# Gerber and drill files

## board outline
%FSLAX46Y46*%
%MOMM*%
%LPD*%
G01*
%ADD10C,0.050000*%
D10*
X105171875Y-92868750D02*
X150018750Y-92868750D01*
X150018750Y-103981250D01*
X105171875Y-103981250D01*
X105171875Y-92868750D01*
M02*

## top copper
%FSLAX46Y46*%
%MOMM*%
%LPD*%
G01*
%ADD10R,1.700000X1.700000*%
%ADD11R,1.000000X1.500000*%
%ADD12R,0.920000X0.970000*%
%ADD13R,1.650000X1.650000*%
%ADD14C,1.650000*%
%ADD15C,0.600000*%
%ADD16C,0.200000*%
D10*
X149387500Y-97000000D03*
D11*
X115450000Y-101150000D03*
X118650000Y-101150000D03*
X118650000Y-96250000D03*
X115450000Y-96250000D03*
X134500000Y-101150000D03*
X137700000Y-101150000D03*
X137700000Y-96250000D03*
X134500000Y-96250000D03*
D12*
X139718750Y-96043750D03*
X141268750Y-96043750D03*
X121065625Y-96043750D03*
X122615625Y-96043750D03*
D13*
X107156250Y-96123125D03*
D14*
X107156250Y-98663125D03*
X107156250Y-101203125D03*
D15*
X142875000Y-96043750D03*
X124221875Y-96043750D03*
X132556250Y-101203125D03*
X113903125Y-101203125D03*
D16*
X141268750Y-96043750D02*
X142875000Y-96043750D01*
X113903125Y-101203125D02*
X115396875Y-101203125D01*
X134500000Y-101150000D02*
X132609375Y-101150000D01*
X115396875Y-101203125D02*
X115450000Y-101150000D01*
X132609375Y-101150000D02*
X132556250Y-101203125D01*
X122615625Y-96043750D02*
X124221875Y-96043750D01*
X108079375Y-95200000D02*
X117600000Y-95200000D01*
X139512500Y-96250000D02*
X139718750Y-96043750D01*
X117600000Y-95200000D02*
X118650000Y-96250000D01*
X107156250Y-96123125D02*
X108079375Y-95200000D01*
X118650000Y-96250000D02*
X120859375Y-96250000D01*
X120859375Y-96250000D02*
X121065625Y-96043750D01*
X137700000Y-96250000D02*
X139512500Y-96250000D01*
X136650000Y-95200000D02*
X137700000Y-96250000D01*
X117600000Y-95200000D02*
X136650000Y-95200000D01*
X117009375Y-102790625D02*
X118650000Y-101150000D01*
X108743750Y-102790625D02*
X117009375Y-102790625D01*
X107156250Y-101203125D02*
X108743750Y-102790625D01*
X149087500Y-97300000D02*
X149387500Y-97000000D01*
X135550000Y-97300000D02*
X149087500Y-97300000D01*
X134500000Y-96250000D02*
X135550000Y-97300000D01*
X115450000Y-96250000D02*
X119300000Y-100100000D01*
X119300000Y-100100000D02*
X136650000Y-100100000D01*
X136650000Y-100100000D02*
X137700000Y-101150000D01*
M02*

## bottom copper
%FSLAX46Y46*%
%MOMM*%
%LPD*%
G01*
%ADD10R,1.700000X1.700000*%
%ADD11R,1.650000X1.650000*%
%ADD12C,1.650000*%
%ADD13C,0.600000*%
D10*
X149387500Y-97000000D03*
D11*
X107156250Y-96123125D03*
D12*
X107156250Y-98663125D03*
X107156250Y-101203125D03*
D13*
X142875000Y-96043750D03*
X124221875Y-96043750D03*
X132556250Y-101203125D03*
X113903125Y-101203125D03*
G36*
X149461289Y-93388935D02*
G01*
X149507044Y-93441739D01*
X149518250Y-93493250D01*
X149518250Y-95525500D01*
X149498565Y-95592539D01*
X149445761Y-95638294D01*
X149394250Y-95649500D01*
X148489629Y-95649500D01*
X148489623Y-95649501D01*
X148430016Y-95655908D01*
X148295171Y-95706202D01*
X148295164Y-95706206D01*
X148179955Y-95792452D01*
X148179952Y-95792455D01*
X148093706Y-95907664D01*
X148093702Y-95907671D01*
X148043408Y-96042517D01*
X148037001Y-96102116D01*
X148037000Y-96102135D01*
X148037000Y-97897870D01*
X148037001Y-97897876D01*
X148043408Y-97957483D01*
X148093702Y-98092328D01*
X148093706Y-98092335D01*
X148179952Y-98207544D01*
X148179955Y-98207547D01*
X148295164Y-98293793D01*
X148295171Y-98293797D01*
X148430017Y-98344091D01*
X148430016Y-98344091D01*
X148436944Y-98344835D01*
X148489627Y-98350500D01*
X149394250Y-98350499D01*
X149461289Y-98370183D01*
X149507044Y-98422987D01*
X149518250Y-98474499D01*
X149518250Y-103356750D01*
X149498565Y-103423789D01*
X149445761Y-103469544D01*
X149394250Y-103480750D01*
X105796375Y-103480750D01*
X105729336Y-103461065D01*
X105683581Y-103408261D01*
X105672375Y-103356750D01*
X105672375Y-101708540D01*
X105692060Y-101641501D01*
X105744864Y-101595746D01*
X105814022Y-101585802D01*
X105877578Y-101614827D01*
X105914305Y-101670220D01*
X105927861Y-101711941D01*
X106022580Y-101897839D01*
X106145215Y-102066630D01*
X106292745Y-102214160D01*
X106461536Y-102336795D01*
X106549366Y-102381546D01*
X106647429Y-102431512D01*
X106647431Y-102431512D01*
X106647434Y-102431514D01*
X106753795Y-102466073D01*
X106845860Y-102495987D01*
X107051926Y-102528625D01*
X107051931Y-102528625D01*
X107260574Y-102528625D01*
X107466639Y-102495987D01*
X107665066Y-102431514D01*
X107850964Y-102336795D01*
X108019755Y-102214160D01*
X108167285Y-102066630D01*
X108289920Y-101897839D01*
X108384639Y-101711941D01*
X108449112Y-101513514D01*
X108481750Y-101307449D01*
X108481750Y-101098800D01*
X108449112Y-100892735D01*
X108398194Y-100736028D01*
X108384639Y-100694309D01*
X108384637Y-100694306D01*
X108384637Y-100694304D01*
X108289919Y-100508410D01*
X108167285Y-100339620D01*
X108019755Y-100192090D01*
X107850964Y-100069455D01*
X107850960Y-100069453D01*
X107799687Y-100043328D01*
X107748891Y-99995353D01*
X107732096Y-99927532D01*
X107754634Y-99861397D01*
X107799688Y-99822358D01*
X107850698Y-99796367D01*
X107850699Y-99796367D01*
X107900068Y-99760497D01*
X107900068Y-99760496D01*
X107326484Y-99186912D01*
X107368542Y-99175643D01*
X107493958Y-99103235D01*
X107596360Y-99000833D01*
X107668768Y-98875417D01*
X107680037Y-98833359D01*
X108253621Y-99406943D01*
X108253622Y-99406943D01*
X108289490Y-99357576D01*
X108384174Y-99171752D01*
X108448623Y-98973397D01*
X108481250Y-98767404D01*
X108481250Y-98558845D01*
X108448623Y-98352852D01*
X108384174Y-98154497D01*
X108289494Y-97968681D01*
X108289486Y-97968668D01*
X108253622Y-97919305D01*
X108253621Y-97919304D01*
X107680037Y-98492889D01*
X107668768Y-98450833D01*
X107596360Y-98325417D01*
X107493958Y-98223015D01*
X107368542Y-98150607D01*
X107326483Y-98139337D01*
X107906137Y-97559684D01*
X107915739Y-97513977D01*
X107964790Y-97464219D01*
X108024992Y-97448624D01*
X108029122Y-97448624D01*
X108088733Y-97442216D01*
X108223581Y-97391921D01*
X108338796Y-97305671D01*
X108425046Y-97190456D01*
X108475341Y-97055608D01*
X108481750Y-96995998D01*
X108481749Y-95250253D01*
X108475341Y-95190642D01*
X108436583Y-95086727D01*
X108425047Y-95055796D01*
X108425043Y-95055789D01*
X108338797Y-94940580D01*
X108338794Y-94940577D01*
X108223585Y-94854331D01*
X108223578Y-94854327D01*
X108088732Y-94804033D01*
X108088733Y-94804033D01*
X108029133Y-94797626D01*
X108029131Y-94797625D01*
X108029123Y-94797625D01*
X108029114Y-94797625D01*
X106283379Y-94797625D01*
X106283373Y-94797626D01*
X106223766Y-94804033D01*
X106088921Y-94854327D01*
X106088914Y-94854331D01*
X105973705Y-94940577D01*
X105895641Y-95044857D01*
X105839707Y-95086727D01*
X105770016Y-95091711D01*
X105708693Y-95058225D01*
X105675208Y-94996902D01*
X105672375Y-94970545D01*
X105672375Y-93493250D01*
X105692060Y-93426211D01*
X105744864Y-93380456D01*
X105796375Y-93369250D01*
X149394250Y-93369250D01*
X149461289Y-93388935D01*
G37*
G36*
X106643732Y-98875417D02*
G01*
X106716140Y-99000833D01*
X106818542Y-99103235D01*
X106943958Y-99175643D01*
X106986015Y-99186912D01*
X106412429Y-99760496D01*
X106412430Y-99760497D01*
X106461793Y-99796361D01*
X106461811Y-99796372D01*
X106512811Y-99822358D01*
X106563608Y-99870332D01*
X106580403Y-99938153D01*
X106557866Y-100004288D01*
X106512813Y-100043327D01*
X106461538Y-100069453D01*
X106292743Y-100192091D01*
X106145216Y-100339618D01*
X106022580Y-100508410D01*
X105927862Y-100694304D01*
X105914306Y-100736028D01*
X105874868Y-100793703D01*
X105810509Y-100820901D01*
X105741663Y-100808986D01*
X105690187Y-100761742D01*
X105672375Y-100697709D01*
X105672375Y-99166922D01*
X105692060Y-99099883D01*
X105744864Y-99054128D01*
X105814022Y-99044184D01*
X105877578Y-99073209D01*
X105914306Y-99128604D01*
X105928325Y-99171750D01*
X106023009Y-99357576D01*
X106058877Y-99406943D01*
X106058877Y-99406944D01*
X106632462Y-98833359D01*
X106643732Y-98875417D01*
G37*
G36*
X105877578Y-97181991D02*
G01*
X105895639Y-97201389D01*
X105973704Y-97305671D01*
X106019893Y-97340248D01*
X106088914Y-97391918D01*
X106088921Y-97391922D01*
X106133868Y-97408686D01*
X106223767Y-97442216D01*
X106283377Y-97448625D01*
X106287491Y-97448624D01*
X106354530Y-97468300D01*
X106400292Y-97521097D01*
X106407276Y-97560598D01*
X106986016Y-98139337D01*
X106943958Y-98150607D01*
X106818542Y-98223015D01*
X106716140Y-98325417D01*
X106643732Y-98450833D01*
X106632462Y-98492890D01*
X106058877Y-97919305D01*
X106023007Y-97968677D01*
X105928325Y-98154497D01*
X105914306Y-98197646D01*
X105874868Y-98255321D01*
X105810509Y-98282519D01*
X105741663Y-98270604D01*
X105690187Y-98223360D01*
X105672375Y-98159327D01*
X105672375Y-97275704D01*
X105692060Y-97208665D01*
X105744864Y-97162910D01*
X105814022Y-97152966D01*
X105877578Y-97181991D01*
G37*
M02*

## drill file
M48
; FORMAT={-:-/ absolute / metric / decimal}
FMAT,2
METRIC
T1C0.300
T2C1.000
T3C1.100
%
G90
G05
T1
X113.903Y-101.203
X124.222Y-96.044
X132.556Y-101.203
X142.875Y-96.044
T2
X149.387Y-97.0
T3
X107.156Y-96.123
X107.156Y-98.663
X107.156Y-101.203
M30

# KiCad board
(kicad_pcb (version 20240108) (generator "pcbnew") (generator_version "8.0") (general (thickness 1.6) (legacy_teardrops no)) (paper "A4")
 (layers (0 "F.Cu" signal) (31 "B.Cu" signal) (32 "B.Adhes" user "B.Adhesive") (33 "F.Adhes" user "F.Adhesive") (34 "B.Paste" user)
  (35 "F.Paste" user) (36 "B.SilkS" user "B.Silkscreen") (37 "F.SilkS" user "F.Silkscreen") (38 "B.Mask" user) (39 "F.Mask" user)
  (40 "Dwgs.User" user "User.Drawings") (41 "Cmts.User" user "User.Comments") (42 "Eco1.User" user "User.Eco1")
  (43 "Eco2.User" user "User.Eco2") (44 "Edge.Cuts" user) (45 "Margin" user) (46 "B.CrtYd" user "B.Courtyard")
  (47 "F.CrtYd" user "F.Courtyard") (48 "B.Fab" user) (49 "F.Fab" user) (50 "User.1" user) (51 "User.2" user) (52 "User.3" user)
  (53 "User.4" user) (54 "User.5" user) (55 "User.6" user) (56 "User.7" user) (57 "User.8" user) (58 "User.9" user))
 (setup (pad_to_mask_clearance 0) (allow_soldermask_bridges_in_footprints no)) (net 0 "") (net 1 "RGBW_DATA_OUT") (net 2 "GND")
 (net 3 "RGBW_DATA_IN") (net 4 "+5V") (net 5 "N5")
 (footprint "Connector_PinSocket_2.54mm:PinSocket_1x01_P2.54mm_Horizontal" (layer "F.Cu") (at 149.3875 97 180)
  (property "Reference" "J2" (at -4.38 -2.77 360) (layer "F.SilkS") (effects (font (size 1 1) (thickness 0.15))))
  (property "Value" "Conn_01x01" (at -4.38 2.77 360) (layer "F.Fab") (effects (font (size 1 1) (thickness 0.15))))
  (pad "1" thru_hole rect (at 0 0 180) (size 1.7 1.7) (drill 1) (layers "*.Cu" "*.Mask") (remove_unused_layers no) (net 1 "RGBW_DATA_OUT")))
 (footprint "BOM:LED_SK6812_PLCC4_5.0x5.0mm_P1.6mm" (layer "F.Cu") (at 117.05 98.7 -90)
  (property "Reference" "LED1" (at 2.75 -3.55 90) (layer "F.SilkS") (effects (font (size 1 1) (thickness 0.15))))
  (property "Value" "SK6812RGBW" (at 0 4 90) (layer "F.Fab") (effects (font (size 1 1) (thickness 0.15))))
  (pad "1" smd rect (at 2.45 1.6 270) (size 1.5 1) (layers "F.Cu" "F.Paste" "F.Mask") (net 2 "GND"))
  (pad "2" smd rect (at 2.45 -1.6 270) (size 1.5 1) (layers "F.Cu" "F.Paste" "F.Mask") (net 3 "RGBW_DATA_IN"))
  (pad "3" smd rect (at -2.45 -1.6 270) (size 1.5 1) (layers "F.Cu" "F.Paste" "F.Mask") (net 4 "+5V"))
  (pad "4" smd rect (at -2.45 1.6 270) (size 1.5 1) (layers "F.Cu" "F.Paste" "F.Mask") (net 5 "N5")))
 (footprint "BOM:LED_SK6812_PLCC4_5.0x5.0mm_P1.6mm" (layer "F.Cu") (at 136.1 98.7 -90)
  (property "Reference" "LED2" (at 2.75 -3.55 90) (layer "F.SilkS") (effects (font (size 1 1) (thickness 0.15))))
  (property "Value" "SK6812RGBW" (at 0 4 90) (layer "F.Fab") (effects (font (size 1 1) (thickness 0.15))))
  (pad "1" smd rect (at 2.45 1.6 270) (size 1.5 1) (layers "F.Cu" "F.Paste" "F.Mask") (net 2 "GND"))
  (pad "2" smd rect (at 2.45 -1.6 270) (size 1.5 1) (layers "F.Cu" "F.Paste" "F.Mask") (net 5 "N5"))
  (pad "3" smd rect (at -2.45 -1.6 270) (size 1.5 1) (layers "F.Cu" "F.Paste" "F.Mask") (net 4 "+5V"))
  (pad "4" smd rect (at -2.45 1.6 270) (size 1.5 1) (layers "F.Cu" "F.Paste" "F.Mask") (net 1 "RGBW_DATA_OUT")))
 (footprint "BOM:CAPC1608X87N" (layer "F.Cu") (at 140.49375 96.04375)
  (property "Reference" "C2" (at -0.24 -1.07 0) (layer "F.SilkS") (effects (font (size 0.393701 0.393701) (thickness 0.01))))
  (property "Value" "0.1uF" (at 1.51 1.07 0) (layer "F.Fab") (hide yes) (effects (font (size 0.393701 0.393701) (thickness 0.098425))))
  (pad "1" smd rect (at -0.775 0) (size 0.92 0.97) (layers "F.Cu" "F.Paste" "F.Mask") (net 4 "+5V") (solder_mask_margin 0.102))
  (pad "2" smd rect (at 0.775 0) (size 0.92 0.97) (layers "F.Cu" "F.Paste" "F.Mask") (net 2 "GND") (solder_mask_margin 0.102)))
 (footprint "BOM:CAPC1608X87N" (layer "F.Cu") (at 121.840625 96.04375)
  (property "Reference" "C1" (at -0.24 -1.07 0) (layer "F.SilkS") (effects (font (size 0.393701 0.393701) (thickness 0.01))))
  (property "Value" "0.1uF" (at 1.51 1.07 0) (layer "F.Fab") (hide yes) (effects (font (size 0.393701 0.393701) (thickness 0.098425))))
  (pad "1" smd rect (at -0.775 0) (size 0.92 0.97) (layers "F.Cu" "F.Paste" "F.Mask") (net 4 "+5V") (solder_mask_margin 0.102))
  (pad "2" smd rect (at 0.775 0) (size 0.92 0.97) (layers "F.Cu" "F.Paste" "F.Mask") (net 2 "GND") (solder_mask_margin 0.102)))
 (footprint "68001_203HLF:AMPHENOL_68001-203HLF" (layer "F.Cu") (at 107.15625 98.663125 -90)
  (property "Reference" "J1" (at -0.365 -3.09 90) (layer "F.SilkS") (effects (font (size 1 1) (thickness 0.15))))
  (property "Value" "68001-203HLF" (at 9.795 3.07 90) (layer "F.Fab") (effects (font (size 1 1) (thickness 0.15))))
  (pad "01" thru_hole rect (at -2.54 0 270) (size 1.65 1.65) (drill 1.1) (layers "*.Cu" "*.Mask") (remove_unused_layers no) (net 4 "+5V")
   (solder_mask_margin 0.102))
  (pad "02" thru_hole circle (at 0 0 270) (size 1.65 1.65) (drill 1.1) (layers "*.Cu" "*.Mask") (remove_unused_layers no) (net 2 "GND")
   (solder_mask_margin 0.102))
  (pad "03" thru_hole circle (at 2.54 0 270) (size 1.65 1.65) (drill 1.1) (layers "*.Cu" "*.Mask") (remove_unused_layers no)
   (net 3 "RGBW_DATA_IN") (solder_mask_margin 0.102)))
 (gr_rect (start 105.171875 92.86875) (end 150.01875 103.98125) (stroke (width 0.05) (type default)) (fill none) (layer "Edge.Cuts"))
 (segment (start 141.26875 96.04375) (end 142.875 96.04375) (width 0.2) (layer "F.Cu") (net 2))
 (segment (start 113.903125 101.203125) (end 115.396875 101.203125) (width 0.2) (layer "F.Cu") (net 2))
 (segment (start 134.5 101.15) (end 132.609375 101.15) (width 0.2) (layer "F.Cu") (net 2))
 (segment (start 115.396875 101.203125) (end 115.45 101.15) (width 0.2) (layer "F.Cu") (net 2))
 (segment (start 132.609375 101.15) (end 132.55625 101.203125) (width 0.2) (layer "F.Cu") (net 2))
 (segment (start 122.615625 96.04375) (end 124.221875 96.04375) (width 0.2) (layer "F.Cu") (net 2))
 (via (at 142.875 96.04375) (size 0.6) (drill 0.3) (layers "F.Cu" "B.Cu") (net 2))
 (via (at 124.221875 96.04375) (size 0.6) (drill 0.3) (layers "F.Cu" "B.Cu") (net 2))
 (via (at 132.55625 101.203125) (size 0.6) (drill 0.3) (layers "F.Cu" "B.Cu") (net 2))
 (via (at 113.903125 101.203125) (size 0.6) (drill 0.3) (layers "F.Cu" "B.Cu") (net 2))
 (segment (start 108.079375 95.2) (end 117.6 95.2) (width 0.2) (layer "F.Cu") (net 4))
 (segment (start 139.5125 96.25) (end 139.71875 96.04375) (width 0.2) (layer "F.Cu") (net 4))
 (segment (start 117.6 95.2) (end 118.65 96.25) (width 0.2) (layer "F.Cu") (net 4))
 (segment (start 107.15625 96.123125) (end 108.079375 95.2) (width 0.2) (layer "F.Cu") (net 4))
 (segment (start 118.65 96.25) (end 120.859375 96.25) (width 0.2) (layer "F.Cu") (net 4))
 (segment (start 120.859375 96.25) (end 121.065625 96.04375) (width 0.2) (layer "F.Cu") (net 4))
 (segment (start 137.7 96.25) (end 139.5125 96.25) (width 0.2) (layer "F.Cu") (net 4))
 (segment (start 136.65 95.2) (end 137.7 96.25) (width 0.2) (layer "F.Cu") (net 4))
 (segment (start 117.6 95.2) (end 136.65 95.2) (width 0.2) (layer "F.Cu") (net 4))
 (segment (start 117.009375 102.790625) (end 118.65 101.15) (width 0.2) (layer "F.Cu") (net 3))
 (segment (start 108.74375 102.790625) (end 117.009375 102.790625) (width 0.2) (layer "F.Cu") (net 3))
 (segment (start 107.15625 101.203125) (end 108.74375 102.790625) (width 0.2) (layer "F.Cu") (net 3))
 (segment (start 149.0875 97.3) (end 149.3875 97) (width 0.2) (layer "F.Cu") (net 1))
 (segment (start 135.55 97.3) (end 149.0875 97.3) (width 0.2) (layer "F.Cu") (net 1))
 (segment (start 134.5 96.25) (end 135.55 97.3) (width 0.2) (layer "F.Cu") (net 1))
 (segment (start 115.45 96.25) (end 119.3 100.1) (width 0.2) (layer "F.Cu") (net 5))
 (segment (start 119.3 100.1) (end 136.65 100.1) (width 0.2) (layer "F.Cu") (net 5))
 (segment (start 136.65 100.1) (end 137.7 101.15) (width 0.2) (layer "F.Cu") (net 5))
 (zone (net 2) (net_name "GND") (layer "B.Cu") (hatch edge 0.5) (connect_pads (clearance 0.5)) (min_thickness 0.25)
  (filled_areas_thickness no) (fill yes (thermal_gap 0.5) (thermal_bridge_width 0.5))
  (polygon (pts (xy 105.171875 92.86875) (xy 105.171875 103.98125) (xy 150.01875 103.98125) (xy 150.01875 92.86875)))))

